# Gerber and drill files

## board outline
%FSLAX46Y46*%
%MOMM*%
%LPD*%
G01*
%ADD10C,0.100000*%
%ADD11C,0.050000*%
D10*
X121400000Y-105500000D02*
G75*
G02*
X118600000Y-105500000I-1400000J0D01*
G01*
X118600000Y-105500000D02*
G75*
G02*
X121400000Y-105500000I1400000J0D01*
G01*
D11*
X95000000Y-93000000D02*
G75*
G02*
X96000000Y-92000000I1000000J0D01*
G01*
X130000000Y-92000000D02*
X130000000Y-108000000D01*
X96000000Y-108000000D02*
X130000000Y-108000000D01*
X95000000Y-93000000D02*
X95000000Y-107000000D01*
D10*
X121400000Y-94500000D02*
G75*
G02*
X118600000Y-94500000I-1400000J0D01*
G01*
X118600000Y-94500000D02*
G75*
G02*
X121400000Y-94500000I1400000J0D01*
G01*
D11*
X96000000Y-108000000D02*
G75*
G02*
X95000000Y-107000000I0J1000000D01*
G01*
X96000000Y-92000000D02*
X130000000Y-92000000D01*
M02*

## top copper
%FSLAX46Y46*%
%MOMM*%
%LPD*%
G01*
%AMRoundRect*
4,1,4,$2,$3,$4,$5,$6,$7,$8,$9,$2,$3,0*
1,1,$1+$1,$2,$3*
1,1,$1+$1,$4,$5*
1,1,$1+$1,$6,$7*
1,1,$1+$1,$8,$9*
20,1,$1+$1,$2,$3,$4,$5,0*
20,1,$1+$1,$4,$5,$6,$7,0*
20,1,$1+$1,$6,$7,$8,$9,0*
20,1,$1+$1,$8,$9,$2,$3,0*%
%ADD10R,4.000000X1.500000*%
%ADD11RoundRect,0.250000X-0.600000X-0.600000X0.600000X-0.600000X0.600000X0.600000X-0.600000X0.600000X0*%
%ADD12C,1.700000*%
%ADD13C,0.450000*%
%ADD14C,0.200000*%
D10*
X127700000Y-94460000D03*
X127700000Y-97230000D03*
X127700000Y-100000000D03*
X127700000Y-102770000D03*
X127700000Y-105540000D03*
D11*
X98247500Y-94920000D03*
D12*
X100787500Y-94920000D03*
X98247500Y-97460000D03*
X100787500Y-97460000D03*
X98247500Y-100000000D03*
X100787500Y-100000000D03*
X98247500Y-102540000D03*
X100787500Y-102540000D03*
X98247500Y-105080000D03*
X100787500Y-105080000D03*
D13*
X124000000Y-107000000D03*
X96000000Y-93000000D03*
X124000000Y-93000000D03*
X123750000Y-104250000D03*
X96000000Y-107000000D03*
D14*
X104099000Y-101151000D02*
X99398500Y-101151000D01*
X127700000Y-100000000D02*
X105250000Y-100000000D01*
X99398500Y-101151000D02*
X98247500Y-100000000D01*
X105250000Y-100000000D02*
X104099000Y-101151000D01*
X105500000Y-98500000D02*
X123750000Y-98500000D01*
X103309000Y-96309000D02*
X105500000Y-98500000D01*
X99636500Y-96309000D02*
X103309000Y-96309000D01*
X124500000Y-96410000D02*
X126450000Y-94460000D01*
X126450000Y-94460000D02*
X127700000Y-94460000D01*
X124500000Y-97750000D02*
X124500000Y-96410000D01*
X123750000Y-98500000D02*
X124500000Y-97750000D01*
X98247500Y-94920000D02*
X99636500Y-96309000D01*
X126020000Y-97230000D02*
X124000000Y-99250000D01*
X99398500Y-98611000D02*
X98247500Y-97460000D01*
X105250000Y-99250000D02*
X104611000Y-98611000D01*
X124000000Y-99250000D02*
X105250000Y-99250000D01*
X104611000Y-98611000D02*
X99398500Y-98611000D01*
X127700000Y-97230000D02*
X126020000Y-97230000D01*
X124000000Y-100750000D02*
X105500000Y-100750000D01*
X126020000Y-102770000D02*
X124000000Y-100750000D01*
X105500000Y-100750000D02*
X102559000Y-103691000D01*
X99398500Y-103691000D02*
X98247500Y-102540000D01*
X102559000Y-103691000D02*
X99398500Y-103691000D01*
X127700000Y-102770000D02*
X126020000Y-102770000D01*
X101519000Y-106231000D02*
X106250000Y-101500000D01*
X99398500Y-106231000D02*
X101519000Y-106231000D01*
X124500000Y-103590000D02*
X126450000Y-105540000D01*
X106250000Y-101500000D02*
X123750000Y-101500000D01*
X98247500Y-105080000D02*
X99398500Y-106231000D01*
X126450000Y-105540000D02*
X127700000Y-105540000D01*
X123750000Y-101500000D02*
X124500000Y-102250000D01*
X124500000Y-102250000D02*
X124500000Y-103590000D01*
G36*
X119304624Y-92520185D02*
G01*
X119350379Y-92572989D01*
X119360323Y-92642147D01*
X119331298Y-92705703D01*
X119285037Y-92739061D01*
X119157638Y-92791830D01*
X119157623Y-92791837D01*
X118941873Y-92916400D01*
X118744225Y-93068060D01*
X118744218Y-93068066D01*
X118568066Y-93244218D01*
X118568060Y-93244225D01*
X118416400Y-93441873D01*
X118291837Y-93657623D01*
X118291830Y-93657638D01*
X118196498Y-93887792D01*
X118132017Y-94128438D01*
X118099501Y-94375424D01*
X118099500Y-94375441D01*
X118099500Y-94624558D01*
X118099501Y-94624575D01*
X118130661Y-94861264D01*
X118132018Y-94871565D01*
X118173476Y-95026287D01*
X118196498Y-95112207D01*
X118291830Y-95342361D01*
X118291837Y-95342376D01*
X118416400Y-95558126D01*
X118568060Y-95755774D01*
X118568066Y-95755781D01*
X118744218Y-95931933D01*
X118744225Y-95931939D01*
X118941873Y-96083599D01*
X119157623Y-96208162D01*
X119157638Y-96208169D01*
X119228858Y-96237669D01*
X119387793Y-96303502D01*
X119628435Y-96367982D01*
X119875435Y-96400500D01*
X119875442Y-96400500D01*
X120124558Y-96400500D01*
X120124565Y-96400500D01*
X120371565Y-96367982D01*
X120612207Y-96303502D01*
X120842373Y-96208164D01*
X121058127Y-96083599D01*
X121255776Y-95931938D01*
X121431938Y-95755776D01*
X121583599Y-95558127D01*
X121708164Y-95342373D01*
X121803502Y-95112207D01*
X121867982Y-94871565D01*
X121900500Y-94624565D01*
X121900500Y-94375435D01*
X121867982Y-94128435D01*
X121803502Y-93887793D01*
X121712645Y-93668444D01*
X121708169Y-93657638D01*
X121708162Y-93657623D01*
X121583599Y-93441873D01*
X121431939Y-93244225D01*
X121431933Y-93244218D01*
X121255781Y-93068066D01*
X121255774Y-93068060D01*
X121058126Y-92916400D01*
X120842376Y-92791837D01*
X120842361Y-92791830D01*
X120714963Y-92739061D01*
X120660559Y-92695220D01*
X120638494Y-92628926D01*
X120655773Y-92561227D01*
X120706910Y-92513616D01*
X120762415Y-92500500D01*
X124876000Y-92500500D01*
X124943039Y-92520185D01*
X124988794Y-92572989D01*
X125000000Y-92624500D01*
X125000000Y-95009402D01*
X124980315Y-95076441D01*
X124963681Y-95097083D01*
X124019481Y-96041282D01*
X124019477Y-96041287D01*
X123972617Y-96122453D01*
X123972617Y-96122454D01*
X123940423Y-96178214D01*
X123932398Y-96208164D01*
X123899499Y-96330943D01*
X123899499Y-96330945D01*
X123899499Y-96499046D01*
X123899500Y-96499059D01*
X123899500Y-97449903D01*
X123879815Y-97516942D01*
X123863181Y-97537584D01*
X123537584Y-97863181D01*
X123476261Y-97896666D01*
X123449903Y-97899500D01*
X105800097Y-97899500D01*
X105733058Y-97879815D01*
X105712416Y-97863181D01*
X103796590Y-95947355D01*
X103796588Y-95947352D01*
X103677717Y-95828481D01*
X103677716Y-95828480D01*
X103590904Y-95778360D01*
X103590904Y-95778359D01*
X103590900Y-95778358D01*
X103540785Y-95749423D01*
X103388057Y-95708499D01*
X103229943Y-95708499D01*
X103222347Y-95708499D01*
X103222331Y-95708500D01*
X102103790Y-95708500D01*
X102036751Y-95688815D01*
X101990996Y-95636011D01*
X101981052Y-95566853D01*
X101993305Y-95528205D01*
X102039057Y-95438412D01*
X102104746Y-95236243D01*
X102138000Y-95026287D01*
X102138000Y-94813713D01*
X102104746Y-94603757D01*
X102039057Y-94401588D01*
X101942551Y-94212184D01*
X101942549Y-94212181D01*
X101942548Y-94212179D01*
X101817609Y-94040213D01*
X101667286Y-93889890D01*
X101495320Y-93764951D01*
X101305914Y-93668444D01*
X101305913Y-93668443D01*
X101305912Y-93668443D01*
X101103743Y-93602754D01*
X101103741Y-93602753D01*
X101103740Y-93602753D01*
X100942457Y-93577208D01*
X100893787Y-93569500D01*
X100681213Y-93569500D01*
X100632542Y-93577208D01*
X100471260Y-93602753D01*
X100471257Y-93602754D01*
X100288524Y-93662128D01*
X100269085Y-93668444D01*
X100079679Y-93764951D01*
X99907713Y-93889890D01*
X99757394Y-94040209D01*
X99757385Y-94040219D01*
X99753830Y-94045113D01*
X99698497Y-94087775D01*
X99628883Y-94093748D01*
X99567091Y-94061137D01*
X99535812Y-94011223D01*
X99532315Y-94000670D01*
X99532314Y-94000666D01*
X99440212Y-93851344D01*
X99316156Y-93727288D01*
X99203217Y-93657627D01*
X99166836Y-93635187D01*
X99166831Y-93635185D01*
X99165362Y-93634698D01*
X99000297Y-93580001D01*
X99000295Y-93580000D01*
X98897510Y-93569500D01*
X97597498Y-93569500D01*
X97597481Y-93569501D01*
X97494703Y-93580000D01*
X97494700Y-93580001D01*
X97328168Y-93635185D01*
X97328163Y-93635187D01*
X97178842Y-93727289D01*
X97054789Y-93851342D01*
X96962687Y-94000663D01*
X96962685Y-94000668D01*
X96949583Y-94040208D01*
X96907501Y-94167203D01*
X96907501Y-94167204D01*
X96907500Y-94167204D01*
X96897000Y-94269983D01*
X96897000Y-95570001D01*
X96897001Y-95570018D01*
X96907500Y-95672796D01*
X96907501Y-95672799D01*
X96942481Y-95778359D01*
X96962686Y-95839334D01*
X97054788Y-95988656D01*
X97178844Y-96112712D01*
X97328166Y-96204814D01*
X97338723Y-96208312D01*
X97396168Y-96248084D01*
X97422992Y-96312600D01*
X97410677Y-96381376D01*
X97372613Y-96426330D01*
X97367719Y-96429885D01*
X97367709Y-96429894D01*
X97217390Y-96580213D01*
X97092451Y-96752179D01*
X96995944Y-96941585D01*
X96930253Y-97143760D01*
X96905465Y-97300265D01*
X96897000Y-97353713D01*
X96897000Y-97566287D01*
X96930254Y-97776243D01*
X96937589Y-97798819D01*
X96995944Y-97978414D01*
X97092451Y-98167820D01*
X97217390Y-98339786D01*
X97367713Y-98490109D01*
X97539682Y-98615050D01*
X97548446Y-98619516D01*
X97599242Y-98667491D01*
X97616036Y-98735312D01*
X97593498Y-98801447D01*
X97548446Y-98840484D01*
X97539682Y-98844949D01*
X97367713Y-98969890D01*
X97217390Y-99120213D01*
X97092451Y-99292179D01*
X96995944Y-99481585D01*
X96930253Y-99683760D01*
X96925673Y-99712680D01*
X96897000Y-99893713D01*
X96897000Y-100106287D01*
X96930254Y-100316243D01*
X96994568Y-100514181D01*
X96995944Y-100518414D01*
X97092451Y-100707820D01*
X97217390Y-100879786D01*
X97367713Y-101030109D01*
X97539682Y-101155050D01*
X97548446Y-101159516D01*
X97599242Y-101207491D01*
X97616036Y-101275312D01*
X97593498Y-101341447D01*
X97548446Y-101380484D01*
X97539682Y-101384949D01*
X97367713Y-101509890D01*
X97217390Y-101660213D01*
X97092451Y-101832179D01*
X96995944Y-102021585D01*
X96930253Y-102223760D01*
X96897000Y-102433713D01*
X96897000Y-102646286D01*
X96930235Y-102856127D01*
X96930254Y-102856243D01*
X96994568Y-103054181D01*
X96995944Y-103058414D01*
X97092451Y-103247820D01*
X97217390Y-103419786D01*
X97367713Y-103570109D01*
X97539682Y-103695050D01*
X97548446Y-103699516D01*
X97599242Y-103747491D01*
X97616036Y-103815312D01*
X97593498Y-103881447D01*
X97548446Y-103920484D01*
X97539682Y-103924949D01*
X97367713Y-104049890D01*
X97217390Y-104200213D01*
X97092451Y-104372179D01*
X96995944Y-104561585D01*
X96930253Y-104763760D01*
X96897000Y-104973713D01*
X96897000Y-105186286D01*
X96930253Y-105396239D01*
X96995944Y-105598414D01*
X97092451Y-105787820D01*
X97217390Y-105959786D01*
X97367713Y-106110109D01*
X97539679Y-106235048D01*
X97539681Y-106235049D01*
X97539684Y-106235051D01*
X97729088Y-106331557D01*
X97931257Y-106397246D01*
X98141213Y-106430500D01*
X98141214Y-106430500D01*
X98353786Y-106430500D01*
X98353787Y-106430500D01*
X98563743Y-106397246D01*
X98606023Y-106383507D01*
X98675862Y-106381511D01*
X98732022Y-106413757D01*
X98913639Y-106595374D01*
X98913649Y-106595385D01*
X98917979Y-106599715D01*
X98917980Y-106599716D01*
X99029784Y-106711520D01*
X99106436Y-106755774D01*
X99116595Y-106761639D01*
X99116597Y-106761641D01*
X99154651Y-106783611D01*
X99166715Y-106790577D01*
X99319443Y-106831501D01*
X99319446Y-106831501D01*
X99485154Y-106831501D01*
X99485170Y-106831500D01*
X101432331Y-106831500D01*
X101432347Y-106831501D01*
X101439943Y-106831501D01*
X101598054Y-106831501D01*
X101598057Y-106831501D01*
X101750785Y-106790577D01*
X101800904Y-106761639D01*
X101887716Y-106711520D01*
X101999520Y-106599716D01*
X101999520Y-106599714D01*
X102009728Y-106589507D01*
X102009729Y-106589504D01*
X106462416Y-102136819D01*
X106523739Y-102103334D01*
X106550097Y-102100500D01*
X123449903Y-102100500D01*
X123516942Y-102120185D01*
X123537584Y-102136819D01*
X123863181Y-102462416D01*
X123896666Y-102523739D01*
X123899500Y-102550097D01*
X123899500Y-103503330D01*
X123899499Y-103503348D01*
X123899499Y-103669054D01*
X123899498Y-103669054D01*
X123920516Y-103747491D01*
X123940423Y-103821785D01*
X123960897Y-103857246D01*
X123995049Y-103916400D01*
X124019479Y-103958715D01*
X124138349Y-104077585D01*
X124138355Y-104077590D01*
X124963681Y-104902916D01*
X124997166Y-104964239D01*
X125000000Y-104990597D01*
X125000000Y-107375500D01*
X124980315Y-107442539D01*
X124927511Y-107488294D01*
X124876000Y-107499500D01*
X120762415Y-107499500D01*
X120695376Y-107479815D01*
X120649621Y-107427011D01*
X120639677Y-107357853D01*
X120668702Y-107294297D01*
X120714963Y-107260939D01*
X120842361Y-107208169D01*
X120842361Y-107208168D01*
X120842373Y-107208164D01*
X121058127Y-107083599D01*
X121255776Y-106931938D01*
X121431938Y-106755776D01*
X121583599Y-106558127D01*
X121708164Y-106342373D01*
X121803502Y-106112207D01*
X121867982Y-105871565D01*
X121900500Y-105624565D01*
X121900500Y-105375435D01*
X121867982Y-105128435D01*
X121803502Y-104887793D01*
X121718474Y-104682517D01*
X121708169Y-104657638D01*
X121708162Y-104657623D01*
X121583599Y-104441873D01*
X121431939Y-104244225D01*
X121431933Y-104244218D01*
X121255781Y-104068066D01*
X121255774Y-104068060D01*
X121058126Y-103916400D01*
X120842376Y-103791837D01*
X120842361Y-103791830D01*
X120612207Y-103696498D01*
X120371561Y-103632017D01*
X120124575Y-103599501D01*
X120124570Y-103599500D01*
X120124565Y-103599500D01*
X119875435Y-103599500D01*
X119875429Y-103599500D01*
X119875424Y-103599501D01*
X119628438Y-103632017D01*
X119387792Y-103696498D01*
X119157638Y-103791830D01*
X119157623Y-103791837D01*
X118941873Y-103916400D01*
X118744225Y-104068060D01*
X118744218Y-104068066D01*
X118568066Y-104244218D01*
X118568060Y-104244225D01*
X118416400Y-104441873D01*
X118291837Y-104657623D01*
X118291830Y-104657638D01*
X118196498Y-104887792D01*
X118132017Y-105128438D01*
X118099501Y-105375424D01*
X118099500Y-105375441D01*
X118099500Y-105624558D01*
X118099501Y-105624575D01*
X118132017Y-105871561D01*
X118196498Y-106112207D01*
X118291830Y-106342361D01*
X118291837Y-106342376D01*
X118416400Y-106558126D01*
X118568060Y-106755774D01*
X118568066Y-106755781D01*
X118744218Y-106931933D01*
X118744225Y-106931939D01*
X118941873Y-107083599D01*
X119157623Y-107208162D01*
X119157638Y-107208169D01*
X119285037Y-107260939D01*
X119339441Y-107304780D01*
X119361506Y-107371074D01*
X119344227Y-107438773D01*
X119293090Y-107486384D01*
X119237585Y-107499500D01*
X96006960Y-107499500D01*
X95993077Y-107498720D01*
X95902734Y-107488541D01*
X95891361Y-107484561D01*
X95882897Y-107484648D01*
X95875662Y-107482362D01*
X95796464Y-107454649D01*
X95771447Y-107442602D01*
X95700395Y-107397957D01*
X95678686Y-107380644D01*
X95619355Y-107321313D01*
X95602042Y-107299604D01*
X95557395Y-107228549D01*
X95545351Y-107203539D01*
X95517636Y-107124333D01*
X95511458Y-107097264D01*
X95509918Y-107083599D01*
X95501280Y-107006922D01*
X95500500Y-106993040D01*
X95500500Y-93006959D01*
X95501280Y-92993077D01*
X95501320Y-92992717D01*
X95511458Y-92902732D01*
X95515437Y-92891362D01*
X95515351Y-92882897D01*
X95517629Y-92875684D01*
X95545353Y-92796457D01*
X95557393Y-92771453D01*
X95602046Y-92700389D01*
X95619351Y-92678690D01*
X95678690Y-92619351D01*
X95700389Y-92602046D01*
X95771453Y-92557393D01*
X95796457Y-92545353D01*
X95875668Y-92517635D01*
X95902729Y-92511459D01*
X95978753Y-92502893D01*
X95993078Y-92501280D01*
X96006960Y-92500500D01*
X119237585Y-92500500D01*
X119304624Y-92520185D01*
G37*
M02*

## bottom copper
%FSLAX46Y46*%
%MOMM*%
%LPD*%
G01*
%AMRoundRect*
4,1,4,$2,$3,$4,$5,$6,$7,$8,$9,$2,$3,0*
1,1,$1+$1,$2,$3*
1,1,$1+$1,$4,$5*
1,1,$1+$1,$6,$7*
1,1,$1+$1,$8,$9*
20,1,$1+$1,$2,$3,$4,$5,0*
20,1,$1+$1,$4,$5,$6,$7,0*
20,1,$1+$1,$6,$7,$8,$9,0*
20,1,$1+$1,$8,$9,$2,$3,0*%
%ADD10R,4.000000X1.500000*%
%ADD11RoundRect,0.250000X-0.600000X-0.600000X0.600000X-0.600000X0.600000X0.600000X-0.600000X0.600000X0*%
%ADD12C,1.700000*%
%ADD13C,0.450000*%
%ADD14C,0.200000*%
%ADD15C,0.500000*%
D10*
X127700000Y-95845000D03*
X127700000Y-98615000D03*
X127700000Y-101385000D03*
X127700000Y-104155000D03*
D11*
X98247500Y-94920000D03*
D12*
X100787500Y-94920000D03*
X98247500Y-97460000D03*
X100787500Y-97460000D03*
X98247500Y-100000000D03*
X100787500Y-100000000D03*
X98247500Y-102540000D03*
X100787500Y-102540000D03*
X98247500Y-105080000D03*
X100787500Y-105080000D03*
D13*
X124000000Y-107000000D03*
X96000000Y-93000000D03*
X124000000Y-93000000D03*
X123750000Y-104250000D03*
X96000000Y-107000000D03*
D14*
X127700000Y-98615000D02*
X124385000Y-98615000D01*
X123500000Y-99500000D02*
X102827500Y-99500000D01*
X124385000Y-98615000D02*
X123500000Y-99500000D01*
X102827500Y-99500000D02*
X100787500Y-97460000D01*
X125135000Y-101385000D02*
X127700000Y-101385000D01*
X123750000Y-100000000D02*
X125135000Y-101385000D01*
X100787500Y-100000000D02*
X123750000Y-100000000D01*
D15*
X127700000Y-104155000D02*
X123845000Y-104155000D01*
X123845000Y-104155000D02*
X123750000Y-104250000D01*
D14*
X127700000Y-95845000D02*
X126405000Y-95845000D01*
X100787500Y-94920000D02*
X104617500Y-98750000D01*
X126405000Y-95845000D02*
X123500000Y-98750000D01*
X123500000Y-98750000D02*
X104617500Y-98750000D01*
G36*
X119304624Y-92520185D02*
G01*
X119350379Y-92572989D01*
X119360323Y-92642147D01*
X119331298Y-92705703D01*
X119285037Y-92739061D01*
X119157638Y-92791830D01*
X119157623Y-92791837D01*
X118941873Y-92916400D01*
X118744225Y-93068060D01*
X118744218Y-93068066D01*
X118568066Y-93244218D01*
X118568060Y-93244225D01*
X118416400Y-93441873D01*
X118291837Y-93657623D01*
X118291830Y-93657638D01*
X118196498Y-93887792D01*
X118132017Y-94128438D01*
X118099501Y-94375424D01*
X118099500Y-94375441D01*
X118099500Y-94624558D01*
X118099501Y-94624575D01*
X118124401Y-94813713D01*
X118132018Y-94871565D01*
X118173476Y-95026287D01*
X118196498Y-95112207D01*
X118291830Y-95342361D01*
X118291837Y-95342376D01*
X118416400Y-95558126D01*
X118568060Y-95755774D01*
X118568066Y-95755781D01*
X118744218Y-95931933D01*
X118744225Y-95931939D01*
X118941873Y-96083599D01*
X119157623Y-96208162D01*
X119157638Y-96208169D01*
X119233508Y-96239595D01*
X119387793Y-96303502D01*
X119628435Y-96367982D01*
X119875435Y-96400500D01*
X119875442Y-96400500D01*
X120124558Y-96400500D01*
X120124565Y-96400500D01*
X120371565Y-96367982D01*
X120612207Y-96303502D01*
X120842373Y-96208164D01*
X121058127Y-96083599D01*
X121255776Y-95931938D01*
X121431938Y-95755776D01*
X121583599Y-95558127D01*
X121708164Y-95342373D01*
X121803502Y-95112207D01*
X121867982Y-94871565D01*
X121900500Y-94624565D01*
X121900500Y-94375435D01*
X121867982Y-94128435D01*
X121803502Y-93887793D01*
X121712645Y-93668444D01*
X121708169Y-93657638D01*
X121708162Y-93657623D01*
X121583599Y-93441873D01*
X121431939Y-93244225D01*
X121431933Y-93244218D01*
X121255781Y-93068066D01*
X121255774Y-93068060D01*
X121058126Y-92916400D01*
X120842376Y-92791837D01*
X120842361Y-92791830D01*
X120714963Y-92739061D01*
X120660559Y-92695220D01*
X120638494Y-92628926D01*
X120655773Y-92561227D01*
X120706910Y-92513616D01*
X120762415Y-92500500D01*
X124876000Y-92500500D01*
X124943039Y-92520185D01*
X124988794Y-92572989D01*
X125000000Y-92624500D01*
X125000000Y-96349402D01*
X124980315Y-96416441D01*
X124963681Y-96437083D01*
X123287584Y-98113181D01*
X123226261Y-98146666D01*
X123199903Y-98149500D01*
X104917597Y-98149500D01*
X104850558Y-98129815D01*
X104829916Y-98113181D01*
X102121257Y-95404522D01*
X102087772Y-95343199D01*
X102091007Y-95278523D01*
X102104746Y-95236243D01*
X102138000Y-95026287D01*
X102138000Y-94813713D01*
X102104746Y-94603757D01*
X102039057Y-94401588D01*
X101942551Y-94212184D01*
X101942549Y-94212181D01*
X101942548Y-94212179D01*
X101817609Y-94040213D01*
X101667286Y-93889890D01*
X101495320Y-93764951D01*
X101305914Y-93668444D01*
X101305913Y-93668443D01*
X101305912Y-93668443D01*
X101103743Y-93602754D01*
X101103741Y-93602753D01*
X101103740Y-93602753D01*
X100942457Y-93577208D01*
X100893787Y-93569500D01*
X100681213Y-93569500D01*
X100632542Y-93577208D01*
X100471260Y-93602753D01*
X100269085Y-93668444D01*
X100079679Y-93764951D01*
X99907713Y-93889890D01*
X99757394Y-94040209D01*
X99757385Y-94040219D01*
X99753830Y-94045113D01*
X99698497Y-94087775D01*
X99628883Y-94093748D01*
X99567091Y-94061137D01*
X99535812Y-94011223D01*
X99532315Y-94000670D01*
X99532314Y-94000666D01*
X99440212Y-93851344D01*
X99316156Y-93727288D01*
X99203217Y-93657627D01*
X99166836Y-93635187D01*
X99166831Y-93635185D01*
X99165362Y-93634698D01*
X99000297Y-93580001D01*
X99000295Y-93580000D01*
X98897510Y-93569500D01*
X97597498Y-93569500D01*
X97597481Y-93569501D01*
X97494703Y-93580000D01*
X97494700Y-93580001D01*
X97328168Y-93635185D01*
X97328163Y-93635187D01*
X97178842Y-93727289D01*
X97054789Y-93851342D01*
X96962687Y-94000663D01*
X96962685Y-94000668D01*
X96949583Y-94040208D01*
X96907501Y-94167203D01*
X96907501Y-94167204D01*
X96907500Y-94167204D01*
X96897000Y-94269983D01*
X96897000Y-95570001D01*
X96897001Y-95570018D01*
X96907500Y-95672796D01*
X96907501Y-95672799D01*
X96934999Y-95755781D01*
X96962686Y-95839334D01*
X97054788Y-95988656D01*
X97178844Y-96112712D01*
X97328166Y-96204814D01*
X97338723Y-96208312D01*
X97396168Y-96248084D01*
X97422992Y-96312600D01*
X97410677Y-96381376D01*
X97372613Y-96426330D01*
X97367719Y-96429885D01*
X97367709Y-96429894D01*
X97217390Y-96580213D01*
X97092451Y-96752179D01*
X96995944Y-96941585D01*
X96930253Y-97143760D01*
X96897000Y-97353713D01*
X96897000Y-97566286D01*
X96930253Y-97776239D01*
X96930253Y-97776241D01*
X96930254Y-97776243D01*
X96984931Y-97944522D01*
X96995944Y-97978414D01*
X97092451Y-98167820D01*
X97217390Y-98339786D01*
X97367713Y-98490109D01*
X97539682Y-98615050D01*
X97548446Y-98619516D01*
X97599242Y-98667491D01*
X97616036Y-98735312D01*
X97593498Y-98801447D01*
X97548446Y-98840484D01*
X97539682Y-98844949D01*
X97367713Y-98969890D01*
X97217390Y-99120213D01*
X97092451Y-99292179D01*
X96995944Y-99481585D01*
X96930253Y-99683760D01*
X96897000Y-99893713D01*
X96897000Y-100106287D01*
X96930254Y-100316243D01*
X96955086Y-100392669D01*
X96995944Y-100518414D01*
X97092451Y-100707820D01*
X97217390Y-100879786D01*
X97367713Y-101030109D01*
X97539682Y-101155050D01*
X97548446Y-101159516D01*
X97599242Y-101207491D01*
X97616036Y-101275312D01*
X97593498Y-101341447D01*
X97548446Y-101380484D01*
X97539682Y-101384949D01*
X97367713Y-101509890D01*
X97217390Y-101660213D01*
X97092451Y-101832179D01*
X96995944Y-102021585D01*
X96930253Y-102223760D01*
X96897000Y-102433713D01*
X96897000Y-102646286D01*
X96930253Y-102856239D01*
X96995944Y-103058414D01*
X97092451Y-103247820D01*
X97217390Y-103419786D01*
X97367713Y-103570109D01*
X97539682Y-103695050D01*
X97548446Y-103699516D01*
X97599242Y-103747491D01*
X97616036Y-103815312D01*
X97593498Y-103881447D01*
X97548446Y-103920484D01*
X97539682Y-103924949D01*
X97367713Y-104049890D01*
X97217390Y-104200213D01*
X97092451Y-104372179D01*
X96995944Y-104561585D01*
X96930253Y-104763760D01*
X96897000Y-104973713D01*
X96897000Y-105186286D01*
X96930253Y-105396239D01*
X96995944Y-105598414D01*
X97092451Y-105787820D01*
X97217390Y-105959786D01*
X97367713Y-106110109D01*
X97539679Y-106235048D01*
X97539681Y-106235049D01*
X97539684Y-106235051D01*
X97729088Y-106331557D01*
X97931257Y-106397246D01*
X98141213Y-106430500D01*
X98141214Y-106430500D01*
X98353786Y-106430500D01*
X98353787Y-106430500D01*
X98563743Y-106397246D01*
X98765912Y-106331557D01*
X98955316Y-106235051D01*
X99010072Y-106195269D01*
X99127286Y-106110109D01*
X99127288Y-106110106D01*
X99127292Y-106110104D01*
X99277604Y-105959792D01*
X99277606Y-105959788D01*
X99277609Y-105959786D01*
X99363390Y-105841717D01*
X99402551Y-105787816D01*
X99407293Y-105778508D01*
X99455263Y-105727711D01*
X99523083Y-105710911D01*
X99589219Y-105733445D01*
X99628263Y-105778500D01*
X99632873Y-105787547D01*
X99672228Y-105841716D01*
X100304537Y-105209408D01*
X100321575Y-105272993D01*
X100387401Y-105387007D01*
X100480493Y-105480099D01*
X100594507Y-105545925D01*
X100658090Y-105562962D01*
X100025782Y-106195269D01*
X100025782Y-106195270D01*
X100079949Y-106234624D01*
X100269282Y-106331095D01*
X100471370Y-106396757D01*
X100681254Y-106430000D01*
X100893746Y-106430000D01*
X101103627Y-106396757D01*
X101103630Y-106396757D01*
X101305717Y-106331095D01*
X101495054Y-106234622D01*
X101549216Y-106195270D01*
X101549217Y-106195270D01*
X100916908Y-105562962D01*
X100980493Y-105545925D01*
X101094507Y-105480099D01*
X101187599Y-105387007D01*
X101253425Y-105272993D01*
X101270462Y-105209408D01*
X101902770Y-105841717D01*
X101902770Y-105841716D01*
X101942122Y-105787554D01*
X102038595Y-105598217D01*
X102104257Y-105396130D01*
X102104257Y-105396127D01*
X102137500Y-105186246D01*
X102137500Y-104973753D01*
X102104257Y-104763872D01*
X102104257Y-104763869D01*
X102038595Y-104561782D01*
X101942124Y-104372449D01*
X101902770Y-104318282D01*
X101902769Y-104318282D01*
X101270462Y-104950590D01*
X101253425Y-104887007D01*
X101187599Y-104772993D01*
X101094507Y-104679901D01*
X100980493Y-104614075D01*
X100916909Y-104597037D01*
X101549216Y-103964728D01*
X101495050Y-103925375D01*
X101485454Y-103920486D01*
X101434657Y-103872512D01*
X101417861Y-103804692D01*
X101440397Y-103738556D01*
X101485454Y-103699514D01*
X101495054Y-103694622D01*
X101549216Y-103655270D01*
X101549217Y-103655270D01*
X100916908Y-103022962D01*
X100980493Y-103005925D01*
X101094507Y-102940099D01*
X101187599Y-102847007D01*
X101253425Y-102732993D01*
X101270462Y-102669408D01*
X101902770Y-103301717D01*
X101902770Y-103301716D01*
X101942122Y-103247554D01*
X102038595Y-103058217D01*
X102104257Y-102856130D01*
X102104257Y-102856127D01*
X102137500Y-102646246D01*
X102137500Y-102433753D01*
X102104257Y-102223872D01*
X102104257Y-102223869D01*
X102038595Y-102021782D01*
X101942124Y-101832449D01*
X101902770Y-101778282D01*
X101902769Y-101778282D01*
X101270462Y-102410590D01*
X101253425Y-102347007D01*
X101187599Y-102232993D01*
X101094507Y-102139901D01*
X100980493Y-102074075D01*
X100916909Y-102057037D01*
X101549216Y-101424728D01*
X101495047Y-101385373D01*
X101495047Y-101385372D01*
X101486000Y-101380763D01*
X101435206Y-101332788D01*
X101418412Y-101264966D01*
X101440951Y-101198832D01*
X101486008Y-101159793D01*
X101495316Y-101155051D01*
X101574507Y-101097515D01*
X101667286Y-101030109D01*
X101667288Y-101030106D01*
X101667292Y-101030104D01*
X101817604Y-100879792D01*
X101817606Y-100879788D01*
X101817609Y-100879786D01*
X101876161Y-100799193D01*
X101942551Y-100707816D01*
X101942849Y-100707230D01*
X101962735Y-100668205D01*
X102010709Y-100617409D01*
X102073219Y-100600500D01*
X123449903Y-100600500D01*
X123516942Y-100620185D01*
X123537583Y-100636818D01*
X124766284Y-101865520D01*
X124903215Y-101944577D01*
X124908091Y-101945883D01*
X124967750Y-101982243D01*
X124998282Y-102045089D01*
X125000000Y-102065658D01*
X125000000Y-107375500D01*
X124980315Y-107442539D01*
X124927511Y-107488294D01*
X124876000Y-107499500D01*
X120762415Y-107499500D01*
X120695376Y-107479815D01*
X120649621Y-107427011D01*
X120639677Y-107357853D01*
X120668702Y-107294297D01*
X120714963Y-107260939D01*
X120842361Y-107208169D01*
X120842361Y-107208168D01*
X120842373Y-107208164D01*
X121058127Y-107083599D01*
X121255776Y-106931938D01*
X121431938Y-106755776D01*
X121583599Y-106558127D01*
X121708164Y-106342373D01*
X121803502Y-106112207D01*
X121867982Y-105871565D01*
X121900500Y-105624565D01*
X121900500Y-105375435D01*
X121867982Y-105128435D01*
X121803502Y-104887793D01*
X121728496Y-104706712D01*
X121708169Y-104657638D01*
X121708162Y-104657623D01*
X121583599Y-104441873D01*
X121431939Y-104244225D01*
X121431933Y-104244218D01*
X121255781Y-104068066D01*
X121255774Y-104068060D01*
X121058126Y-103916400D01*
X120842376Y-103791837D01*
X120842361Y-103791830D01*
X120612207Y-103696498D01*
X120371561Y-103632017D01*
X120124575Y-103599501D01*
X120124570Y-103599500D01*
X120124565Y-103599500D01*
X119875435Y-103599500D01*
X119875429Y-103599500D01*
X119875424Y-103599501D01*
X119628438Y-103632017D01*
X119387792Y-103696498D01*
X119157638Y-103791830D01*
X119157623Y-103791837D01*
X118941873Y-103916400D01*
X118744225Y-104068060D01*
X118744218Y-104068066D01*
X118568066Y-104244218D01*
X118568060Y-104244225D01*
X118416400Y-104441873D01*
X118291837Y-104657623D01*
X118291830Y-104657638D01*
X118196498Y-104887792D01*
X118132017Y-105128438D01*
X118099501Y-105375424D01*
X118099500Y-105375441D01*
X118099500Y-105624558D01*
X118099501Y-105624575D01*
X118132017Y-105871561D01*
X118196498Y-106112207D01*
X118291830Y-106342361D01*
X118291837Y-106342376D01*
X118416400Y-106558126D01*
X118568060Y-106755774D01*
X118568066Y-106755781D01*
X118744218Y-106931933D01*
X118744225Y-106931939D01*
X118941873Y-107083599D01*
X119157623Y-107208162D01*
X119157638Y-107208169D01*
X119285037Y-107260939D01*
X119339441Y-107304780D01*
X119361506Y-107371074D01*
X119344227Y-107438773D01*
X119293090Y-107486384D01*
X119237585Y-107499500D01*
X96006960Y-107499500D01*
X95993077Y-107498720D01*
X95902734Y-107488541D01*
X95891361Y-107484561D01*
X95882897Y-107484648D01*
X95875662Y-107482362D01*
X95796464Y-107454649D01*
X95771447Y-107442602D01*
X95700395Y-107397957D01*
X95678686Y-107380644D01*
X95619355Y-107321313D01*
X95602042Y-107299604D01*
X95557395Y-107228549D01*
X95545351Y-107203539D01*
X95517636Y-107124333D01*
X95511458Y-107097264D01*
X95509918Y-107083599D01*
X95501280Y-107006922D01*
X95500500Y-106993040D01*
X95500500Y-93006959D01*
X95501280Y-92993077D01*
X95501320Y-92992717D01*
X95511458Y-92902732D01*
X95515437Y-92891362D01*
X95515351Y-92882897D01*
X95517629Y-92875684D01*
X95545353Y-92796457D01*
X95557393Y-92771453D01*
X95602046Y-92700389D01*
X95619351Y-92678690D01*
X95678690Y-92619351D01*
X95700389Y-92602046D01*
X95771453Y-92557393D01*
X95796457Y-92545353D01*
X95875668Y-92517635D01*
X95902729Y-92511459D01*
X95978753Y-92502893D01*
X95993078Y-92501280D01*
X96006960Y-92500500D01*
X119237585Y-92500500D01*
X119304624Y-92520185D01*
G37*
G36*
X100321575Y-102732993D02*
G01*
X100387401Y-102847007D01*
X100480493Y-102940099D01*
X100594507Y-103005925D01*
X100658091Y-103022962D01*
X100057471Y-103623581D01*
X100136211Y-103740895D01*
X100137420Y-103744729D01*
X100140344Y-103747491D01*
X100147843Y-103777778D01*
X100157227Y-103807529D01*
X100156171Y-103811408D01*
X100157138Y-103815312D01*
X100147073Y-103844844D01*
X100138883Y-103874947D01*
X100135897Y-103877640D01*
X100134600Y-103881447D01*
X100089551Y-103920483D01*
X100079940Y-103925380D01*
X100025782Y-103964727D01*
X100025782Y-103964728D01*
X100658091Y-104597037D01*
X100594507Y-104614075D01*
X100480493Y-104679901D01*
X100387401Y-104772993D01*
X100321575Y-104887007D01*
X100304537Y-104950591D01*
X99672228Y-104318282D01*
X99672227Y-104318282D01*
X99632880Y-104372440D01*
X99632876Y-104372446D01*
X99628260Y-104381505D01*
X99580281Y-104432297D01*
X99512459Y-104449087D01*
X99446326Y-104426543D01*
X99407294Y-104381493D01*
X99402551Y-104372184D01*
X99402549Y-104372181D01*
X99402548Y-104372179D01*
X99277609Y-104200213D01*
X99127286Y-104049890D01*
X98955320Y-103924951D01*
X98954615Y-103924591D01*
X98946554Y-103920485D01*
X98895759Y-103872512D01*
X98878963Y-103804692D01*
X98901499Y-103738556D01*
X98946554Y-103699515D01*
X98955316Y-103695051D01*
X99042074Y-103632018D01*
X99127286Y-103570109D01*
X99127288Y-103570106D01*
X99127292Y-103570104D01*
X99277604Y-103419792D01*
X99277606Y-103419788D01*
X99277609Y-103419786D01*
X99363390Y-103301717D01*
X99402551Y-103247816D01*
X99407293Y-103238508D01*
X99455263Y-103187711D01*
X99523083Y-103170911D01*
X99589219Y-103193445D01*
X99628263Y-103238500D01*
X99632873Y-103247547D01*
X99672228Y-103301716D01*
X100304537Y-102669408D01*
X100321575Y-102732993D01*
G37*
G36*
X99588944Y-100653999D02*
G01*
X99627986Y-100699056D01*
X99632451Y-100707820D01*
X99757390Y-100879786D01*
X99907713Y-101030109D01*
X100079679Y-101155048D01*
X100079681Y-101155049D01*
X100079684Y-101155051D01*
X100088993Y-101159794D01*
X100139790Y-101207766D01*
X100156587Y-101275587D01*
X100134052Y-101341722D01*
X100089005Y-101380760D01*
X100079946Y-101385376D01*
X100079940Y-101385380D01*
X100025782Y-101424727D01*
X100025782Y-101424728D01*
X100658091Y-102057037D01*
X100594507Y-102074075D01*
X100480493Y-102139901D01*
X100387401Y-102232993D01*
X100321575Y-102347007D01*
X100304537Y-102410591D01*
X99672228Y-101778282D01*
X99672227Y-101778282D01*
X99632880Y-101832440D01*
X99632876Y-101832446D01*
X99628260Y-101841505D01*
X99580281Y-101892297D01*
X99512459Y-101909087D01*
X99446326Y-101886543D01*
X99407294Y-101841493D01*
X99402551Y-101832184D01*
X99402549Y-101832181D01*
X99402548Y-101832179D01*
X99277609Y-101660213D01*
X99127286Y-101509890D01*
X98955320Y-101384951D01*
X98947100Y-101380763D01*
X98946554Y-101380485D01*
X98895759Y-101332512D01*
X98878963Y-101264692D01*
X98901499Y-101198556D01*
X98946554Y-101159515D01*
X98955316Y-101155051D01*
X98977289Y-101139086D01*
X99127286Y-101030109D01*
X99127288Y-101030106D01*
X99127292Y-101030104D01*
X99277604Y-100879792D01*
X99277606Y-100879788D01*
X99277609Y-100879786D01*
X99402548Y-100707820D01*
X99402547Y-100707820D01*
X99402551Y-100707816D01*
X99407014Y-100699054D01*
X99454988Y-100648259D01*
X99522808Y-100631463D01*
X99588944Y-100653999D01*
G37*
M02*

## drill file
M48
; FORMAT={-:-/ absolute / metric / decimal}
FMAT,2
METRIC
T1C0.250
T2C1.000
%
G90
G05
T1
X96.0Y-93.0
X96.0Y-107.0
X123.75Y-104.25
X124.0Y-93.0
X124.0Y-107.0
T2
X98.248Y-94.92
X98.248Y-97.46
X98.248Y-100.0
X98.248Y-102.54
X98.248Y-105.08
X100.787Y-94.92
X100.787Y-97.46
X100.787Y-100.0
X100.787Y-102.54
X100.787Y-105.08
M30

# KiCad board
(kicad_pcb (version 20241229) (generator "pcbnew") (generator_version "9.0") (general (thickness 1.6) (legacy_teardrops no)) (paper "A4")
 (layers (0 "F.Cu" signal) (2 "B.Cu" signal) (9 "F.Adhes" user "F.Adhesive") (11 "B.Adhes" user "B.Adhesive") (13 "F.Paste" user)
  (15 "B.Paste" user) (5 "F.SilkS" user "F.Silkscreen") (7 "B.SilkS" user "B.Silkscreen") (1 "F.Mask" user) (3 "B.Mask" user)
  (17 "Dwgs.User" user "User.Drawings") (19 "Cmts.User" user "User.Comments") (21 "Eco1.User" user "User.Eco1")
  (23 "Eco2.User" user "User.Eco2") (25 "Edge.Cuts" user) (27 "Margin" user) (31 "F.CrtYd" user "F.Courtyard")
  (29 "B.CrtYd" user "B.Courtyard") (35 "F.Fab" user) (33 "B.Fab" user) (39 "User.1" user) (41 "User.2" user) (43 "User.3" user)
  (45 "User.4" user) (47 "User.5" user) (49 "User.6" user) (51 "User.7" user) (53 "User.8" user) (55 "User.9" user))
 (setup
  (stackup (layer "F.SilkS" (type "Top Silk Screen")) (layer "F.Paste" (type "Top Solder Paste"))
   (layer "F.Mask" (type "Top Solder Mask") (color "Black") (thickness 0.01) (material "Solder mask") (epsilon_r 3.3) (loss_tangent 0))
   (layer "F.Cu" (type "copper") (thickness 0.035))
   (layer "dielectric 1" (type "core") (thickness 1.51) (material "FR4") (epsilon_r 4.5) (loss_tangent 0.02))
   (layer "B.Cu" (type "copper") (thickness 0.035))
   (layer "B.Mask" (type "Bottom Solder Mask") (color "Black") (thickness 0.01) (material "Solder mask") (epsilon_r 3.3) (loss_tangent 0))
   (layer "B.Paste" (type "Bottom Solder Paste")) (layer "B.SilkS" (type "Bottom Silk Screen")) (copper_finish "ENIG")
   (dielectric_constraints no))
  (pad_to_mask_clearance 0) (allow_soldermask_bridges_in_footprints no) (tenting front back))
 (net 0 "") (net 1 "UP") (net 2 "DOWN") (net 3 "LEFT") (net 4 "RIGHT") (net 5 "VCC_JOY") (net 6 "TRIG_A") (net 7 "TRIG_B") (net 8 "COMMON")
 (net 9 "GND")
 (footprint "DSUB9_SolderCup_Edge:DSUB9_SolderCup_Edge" (layer "F.Cu") (at 130 100 -90)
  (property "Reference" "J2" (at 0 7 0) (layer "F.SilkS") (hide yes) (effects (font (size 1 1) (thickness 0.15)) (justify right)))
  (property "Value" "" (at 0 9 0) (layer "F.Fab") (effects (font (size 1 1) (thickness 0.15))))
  (pad "1" connect rect (at -5.54 2.3 270) (size 1.5 4) (layers "F.Cu" "F.Mask") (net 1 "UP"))
  (pad "2" connect rect (at -2.77 2.3 270) (size 1.5 4) (layers "F.Cu" "F.Mask") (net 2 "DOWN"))
  (pad "3" connect rect (at 0 2.3 270) (size 1.5 4) (layers "F.Cu" "F.Mask") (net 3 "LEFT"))
  (pad "4" connect rect (at 2.77 2.3 270) (size 1.5 4) (layers "F.Cu" "F.Mask") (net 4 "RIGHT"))
  (pad "5" connect rect (at 5.54 2.3 270) (size 1.5 4) (layers "F.Cu" "F.Mask") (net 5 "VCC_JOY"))
  (pad "6" connect rect (at -4.155 2.3 270) (size 1.5 4) (layers "B.Cu" "B.Mask") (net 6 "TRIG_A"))
  (pad "7" connect rect (at -1.385 2.3 270) (size 1.5 4) (layers "B.Cu" "B.Mask") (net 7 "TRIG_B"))
  (pad "8" connect rect (at 1.385 2.3 270) (size 1.5 4) (layers "B.Cu" "B.Mask") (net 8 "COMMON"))
  (pad "9" connect rect (at 4.155 2.3 270) (size 1.5 4) (layers "B.Cu" "B.Mask") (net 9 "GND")))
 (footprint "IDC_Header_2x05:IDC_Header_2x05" (layer "F.Cu") (at 98.2475 94.92)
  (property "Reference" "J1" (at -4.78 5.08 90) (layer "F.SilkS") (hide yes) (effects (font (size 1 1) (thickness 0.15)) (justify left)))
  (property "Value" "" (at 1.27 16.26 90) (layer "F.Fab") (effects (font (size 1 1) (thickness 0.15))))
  (pad "1" thru_hole roundrect (at 0 0) (size 1.7 1.7) (drill 1) (layers "*.Cu" "*.Mask") (remove_unused_layers no)
   (roundrect_rratio 0.147059) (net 1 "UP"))
  (pad "2" thru_hole circle (at 2.54 0) (size 1.7 1.7) (drill 1) (layers "*.Cu" "*.Mask") (remove_unused_layers no) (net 6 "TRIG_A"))
  (pad "3" thru_hole circle (at 0 2.54) (size 1.7 1.7) (drill 1) (layers "*.Cu" "*.Mask") (remove_unused_layers no) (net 2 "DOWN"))
  (pad "4" thru_hole circle (at 2.54 2.54) (size 1.7 1.7) (drill 1) (layers "*.Cu" "*.Mask") (remove_unused_layers no) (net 7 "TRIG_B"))
  (pad "5" thru_hole circle (at 0 5.08) (size 1.7 1.7) (drill 1) (layers "*.Cu" "*.Mask") (remove_unused_layers no) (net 3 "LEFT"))
  (pad "6" thru_hole circle (at 2.54 5.08) (size 1.7 1.7) (drill 1) (layers "*.Cu" "*.Mask") (remove_unused_layers no) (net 8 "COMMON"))
  (pad "7" thru_hole circle (at 0 7.62) (size 1.7 1.7) (drill 1) (layers "*.Cu" "*.Mask") (remove_unused_layers no) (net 4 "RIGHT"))
  (pad "8" thru_hole circle (at 2.54 7.62) (size 1.7 1.7) (drill 1) (layers "*.Cu" "*.Mask") (remove_unused_layers no) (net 9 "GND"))
  (pad "9" thru_hole circle (at 0 10.16) (size 1.7 1.7) (drill 1) (layers "*.Cu" "*.Mask") (remove_unused_layers no) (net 5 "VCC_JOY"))
  (pad "10" thru_hole circle (at 2.54 10.16) (size 1.7 1.7) (drill 1) (layers "*.Cu" "*.Mask") (remove_unused_layers no) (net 9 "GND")))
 (gr_circle (center 120 105.5) (end 120 106.9) (stroke (width 0.1) (type solid)) (fill no) (layer "Edge.Cuts"))
 (gr_arc (start 95 93) (mid 95.292893 92.292893) (end 96 92) (stroke (width 0.05) (type default)) (layer "Edge.Cuts"))
 (gr_line (start 130 92) (end 130 108) (stroke (width 0.05) (type default)) (layer "Edge.Cuts"))
 (gr_line (start 96 108) (end 130 108) (stroke (width 0.05) (type default)) (layer "Edge.Cuts"))
 (gr_line (start 95 93) (end 95 107) (stroke (width 0.05) (type default)) (layer "Edge.Cuts"))
 (gr_circle (center 120 94.5) (end 120 95.9) (stroke (width 0.1) (type solid)) (fill no) (layer "Edge.Cuts"))
 (gr_arc (start 96 108) (mid 95.292893 107.707107) (end 95 107) (stroke (width 0.05) (type default)) (layer "Edge.Cuts"))
 (gr_line (start 96 92) (end 130 92) (stroke (width 0.05) (type default)) (layer "Edge.Cuts"))
 (segment (start 127.7 98.615) (end 124.385 98.615) (width 0.2) (layer "B.Cu") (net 7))
 (segment (start 123.5 99.5) (end 102.8275 99.5) (width 0.2) (layer "B.Cu") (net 7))
 (segment (start 124.385 98.615) (end 123.5 99.5) (width 0.2) (layer "B.Cu") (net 7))
 (segment (start 102.8275 99.5) (end 100.7875 97.46) (width 0.2) (layer "B.Cu") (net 7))
 (segment (start 104.099 101.151) (end 99.3985 101.151) (width 0.2) (layer "F.Cu") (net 3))
 (segment (start 127.7 100) (end 105.25 100) (width 0.2) (layer "F.Cu") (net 3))
 (segment (start 99.3985 101.151) (end 98.2475 100) (width 0.2) (layer "F.Cu") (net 3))
 (segment (start 105.25 100) (end 104.099 101.151) (width 0.2) (layer "F.Cu") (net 3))
 (segment (start 125.135 101.385) (end 127.7 101.385) (width 0.2) (layer "B.Cu") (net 8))
 (segment (start 123.75 100) (end 125.135 101.385) (width 0.2) (layer "B.Cu") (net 8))
 (segment (start 100.7875 100) (end 123.75 100) (width 0.2) (layer "B.Cu") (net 8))
 (via (at 124 107) (size 0.45) (drill 0.25) (layers "F.Cu" "B.Cu") (free yes) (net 9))
 (via (at 96 93) (size 0.45) (drill 0.25) (layers "F.Cu" "B.Cu") (free yes) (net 9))
 (via (at 124 93) (size 0.45) (drill 0.25) (layers "F.Cu" "B.Cu") (free yes) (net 9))
 (via (at 123.75 104.25) (size 0.45) (drill 0.25) (layers "F.Cu" "B.Cu") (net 9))
 (via (at 96 107) (size 0.45) (drill 0.25) (layers "F.Cu" "B.Cu") (free yes) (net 9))
 (segment (start 127.7 104.155) (end 123.845 104.155) (width 0.5) (layer "B.Cu") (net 9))
 (segment (start 123.845 104.155) (end 123.75 104.25) (width 0.5) (layer "B.Cu") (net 9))
 (segment (start 105.5 98.5) (end 123.75 98.5) (width 0.2) (layer "F.Cu") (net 1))
 (segment (start 103.309 96.309) (end 105.5 98.5) (width 0.2) (layer "F.Cu") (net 1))
 (segment (start 99.6365 96.309) (end 103.309 96.309) (width 0.2) (layer "F.Cu") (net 1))
 (segment (start 124.5 96.41) (end 126.45 94.46) (width 0.2) (layer "F.Cu") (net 1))
 (segment (start 126.45 94.46) (end 127.7 94.46) (width 0.2) (layer "F.Cu") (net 1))
 (segment (start 124.5 97.75) (end 124.5 96.41) (width 0.2) (layer "F.Cu") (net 1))
 (segment (start 123.75 98.5) (end 124.5 97.75) (width 0.2) (layer "F.Cu") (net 1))
 (segment (start 98.2475 94.92) (end 99.6365 96.309) (width 0.2) (layer "F.Cu") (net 1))
 (segment (start 126.02 97.23) (end 124 99.25) (width 0.2) (layer "F.Cu") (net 2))
 (segment (start 99.3985 98.611) (end 98.2475 97.46) (width 0.2) (layer "F.Cu") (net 2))
 (segment (start 105.25 99.25) (end 104.611 98.611) (width 0.2) (layer "F.Cu") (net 2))
 (segment (start 124 99.25) (end 105.25 99.25) (width 0.2) (layer "F.Cu") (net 2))
 (segment (start 104.611 98.611) (end 99.3985 98.611) (width 0.2) (layer "F.Cu") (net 2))
 (segment (start 127.7 97.23) (end 126.02 97.23) (width 0.2) (layer "F.Cu") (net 2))
 (segment (start 124 100.75) (end 105.5 100.75) (width 0.2) (layer "F.Cu") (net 4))
 (segment (start 126.02 102.77) (end 124 100.75) (width 0.2) (layer "F.Cu") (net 4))
 (segment (start 105.5 100.75) (end 102.559 103.691) (width 0.2) (layer "F.Cu") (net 4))
 (segment (start 99.3985 103.691) (end 98.2475 102.54) (width 0.2) (layer "F.Cu") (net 4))
 (segment (start 102.559 103.691) (end 99.3985 103.691) (width 0.2) (layer "F.Cu") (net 4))
 (segment (start 127.7 102.77) (end 126.02 102.77) (width 0.2) (layer "F.Cu") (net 4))
 (segment (start 101.519 106.231) (end 106.25 101.5) (width 0.2) (layer "F.Cu") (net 5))
 (segment (start 99.3985 106.231) (end 101.519 106.231) (width 0.2) (layer "F.Cu") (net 5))
 (segment (start 124.5 103.59) (end 126.45 105.54) (width 0.2) (layer "F.Cu") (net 5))
 (segment (start 106.25 101.5) (end 123.75 101.5) (width 0.2) (layer "F.Cu") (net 5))
 (segment (start 98.2475 105.08) (end 99.3985 106.231) (width 0.2) (layer "F.Cu") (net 5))
 (segment (start 126.45 105.54) (end 127.7 105.54) (width 0.2) (layer "F.Cu") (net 5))
 (segment (start 123.75 101.5) (end 124.5 102.25) (width 0.2) (layer "F.Cu") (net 5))
 (segment (start 124.5 102.25) (end 124.5 103.59) (width 0.2) (layer "F.Cu") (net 5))
 (segment (start 127.7 95.845) (end 126.405 95.845) (width 0.2) (layer "B.Cu") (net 6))
 (segment (start 100.7875 94.92) (end 104.6175 98.75) (width 0.2) (layer "B.Cu") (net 6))
 (segment (start 126.405 95.845) (end 123.5 98.75) (width 0.2) (layer "B.Cu") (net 6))
 (segment (start 123.5 98.75) (end 104.6175 98.75) (width 0.2) (layer "B.Cu") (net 6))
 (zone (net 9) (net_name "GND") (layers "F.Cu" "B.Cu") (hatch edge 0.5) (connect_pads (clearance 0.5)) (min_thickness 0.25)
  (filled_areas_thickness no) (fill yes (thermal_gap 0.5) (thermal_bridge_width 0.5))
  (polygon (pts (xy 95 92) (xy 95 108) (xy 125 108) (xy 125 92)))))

